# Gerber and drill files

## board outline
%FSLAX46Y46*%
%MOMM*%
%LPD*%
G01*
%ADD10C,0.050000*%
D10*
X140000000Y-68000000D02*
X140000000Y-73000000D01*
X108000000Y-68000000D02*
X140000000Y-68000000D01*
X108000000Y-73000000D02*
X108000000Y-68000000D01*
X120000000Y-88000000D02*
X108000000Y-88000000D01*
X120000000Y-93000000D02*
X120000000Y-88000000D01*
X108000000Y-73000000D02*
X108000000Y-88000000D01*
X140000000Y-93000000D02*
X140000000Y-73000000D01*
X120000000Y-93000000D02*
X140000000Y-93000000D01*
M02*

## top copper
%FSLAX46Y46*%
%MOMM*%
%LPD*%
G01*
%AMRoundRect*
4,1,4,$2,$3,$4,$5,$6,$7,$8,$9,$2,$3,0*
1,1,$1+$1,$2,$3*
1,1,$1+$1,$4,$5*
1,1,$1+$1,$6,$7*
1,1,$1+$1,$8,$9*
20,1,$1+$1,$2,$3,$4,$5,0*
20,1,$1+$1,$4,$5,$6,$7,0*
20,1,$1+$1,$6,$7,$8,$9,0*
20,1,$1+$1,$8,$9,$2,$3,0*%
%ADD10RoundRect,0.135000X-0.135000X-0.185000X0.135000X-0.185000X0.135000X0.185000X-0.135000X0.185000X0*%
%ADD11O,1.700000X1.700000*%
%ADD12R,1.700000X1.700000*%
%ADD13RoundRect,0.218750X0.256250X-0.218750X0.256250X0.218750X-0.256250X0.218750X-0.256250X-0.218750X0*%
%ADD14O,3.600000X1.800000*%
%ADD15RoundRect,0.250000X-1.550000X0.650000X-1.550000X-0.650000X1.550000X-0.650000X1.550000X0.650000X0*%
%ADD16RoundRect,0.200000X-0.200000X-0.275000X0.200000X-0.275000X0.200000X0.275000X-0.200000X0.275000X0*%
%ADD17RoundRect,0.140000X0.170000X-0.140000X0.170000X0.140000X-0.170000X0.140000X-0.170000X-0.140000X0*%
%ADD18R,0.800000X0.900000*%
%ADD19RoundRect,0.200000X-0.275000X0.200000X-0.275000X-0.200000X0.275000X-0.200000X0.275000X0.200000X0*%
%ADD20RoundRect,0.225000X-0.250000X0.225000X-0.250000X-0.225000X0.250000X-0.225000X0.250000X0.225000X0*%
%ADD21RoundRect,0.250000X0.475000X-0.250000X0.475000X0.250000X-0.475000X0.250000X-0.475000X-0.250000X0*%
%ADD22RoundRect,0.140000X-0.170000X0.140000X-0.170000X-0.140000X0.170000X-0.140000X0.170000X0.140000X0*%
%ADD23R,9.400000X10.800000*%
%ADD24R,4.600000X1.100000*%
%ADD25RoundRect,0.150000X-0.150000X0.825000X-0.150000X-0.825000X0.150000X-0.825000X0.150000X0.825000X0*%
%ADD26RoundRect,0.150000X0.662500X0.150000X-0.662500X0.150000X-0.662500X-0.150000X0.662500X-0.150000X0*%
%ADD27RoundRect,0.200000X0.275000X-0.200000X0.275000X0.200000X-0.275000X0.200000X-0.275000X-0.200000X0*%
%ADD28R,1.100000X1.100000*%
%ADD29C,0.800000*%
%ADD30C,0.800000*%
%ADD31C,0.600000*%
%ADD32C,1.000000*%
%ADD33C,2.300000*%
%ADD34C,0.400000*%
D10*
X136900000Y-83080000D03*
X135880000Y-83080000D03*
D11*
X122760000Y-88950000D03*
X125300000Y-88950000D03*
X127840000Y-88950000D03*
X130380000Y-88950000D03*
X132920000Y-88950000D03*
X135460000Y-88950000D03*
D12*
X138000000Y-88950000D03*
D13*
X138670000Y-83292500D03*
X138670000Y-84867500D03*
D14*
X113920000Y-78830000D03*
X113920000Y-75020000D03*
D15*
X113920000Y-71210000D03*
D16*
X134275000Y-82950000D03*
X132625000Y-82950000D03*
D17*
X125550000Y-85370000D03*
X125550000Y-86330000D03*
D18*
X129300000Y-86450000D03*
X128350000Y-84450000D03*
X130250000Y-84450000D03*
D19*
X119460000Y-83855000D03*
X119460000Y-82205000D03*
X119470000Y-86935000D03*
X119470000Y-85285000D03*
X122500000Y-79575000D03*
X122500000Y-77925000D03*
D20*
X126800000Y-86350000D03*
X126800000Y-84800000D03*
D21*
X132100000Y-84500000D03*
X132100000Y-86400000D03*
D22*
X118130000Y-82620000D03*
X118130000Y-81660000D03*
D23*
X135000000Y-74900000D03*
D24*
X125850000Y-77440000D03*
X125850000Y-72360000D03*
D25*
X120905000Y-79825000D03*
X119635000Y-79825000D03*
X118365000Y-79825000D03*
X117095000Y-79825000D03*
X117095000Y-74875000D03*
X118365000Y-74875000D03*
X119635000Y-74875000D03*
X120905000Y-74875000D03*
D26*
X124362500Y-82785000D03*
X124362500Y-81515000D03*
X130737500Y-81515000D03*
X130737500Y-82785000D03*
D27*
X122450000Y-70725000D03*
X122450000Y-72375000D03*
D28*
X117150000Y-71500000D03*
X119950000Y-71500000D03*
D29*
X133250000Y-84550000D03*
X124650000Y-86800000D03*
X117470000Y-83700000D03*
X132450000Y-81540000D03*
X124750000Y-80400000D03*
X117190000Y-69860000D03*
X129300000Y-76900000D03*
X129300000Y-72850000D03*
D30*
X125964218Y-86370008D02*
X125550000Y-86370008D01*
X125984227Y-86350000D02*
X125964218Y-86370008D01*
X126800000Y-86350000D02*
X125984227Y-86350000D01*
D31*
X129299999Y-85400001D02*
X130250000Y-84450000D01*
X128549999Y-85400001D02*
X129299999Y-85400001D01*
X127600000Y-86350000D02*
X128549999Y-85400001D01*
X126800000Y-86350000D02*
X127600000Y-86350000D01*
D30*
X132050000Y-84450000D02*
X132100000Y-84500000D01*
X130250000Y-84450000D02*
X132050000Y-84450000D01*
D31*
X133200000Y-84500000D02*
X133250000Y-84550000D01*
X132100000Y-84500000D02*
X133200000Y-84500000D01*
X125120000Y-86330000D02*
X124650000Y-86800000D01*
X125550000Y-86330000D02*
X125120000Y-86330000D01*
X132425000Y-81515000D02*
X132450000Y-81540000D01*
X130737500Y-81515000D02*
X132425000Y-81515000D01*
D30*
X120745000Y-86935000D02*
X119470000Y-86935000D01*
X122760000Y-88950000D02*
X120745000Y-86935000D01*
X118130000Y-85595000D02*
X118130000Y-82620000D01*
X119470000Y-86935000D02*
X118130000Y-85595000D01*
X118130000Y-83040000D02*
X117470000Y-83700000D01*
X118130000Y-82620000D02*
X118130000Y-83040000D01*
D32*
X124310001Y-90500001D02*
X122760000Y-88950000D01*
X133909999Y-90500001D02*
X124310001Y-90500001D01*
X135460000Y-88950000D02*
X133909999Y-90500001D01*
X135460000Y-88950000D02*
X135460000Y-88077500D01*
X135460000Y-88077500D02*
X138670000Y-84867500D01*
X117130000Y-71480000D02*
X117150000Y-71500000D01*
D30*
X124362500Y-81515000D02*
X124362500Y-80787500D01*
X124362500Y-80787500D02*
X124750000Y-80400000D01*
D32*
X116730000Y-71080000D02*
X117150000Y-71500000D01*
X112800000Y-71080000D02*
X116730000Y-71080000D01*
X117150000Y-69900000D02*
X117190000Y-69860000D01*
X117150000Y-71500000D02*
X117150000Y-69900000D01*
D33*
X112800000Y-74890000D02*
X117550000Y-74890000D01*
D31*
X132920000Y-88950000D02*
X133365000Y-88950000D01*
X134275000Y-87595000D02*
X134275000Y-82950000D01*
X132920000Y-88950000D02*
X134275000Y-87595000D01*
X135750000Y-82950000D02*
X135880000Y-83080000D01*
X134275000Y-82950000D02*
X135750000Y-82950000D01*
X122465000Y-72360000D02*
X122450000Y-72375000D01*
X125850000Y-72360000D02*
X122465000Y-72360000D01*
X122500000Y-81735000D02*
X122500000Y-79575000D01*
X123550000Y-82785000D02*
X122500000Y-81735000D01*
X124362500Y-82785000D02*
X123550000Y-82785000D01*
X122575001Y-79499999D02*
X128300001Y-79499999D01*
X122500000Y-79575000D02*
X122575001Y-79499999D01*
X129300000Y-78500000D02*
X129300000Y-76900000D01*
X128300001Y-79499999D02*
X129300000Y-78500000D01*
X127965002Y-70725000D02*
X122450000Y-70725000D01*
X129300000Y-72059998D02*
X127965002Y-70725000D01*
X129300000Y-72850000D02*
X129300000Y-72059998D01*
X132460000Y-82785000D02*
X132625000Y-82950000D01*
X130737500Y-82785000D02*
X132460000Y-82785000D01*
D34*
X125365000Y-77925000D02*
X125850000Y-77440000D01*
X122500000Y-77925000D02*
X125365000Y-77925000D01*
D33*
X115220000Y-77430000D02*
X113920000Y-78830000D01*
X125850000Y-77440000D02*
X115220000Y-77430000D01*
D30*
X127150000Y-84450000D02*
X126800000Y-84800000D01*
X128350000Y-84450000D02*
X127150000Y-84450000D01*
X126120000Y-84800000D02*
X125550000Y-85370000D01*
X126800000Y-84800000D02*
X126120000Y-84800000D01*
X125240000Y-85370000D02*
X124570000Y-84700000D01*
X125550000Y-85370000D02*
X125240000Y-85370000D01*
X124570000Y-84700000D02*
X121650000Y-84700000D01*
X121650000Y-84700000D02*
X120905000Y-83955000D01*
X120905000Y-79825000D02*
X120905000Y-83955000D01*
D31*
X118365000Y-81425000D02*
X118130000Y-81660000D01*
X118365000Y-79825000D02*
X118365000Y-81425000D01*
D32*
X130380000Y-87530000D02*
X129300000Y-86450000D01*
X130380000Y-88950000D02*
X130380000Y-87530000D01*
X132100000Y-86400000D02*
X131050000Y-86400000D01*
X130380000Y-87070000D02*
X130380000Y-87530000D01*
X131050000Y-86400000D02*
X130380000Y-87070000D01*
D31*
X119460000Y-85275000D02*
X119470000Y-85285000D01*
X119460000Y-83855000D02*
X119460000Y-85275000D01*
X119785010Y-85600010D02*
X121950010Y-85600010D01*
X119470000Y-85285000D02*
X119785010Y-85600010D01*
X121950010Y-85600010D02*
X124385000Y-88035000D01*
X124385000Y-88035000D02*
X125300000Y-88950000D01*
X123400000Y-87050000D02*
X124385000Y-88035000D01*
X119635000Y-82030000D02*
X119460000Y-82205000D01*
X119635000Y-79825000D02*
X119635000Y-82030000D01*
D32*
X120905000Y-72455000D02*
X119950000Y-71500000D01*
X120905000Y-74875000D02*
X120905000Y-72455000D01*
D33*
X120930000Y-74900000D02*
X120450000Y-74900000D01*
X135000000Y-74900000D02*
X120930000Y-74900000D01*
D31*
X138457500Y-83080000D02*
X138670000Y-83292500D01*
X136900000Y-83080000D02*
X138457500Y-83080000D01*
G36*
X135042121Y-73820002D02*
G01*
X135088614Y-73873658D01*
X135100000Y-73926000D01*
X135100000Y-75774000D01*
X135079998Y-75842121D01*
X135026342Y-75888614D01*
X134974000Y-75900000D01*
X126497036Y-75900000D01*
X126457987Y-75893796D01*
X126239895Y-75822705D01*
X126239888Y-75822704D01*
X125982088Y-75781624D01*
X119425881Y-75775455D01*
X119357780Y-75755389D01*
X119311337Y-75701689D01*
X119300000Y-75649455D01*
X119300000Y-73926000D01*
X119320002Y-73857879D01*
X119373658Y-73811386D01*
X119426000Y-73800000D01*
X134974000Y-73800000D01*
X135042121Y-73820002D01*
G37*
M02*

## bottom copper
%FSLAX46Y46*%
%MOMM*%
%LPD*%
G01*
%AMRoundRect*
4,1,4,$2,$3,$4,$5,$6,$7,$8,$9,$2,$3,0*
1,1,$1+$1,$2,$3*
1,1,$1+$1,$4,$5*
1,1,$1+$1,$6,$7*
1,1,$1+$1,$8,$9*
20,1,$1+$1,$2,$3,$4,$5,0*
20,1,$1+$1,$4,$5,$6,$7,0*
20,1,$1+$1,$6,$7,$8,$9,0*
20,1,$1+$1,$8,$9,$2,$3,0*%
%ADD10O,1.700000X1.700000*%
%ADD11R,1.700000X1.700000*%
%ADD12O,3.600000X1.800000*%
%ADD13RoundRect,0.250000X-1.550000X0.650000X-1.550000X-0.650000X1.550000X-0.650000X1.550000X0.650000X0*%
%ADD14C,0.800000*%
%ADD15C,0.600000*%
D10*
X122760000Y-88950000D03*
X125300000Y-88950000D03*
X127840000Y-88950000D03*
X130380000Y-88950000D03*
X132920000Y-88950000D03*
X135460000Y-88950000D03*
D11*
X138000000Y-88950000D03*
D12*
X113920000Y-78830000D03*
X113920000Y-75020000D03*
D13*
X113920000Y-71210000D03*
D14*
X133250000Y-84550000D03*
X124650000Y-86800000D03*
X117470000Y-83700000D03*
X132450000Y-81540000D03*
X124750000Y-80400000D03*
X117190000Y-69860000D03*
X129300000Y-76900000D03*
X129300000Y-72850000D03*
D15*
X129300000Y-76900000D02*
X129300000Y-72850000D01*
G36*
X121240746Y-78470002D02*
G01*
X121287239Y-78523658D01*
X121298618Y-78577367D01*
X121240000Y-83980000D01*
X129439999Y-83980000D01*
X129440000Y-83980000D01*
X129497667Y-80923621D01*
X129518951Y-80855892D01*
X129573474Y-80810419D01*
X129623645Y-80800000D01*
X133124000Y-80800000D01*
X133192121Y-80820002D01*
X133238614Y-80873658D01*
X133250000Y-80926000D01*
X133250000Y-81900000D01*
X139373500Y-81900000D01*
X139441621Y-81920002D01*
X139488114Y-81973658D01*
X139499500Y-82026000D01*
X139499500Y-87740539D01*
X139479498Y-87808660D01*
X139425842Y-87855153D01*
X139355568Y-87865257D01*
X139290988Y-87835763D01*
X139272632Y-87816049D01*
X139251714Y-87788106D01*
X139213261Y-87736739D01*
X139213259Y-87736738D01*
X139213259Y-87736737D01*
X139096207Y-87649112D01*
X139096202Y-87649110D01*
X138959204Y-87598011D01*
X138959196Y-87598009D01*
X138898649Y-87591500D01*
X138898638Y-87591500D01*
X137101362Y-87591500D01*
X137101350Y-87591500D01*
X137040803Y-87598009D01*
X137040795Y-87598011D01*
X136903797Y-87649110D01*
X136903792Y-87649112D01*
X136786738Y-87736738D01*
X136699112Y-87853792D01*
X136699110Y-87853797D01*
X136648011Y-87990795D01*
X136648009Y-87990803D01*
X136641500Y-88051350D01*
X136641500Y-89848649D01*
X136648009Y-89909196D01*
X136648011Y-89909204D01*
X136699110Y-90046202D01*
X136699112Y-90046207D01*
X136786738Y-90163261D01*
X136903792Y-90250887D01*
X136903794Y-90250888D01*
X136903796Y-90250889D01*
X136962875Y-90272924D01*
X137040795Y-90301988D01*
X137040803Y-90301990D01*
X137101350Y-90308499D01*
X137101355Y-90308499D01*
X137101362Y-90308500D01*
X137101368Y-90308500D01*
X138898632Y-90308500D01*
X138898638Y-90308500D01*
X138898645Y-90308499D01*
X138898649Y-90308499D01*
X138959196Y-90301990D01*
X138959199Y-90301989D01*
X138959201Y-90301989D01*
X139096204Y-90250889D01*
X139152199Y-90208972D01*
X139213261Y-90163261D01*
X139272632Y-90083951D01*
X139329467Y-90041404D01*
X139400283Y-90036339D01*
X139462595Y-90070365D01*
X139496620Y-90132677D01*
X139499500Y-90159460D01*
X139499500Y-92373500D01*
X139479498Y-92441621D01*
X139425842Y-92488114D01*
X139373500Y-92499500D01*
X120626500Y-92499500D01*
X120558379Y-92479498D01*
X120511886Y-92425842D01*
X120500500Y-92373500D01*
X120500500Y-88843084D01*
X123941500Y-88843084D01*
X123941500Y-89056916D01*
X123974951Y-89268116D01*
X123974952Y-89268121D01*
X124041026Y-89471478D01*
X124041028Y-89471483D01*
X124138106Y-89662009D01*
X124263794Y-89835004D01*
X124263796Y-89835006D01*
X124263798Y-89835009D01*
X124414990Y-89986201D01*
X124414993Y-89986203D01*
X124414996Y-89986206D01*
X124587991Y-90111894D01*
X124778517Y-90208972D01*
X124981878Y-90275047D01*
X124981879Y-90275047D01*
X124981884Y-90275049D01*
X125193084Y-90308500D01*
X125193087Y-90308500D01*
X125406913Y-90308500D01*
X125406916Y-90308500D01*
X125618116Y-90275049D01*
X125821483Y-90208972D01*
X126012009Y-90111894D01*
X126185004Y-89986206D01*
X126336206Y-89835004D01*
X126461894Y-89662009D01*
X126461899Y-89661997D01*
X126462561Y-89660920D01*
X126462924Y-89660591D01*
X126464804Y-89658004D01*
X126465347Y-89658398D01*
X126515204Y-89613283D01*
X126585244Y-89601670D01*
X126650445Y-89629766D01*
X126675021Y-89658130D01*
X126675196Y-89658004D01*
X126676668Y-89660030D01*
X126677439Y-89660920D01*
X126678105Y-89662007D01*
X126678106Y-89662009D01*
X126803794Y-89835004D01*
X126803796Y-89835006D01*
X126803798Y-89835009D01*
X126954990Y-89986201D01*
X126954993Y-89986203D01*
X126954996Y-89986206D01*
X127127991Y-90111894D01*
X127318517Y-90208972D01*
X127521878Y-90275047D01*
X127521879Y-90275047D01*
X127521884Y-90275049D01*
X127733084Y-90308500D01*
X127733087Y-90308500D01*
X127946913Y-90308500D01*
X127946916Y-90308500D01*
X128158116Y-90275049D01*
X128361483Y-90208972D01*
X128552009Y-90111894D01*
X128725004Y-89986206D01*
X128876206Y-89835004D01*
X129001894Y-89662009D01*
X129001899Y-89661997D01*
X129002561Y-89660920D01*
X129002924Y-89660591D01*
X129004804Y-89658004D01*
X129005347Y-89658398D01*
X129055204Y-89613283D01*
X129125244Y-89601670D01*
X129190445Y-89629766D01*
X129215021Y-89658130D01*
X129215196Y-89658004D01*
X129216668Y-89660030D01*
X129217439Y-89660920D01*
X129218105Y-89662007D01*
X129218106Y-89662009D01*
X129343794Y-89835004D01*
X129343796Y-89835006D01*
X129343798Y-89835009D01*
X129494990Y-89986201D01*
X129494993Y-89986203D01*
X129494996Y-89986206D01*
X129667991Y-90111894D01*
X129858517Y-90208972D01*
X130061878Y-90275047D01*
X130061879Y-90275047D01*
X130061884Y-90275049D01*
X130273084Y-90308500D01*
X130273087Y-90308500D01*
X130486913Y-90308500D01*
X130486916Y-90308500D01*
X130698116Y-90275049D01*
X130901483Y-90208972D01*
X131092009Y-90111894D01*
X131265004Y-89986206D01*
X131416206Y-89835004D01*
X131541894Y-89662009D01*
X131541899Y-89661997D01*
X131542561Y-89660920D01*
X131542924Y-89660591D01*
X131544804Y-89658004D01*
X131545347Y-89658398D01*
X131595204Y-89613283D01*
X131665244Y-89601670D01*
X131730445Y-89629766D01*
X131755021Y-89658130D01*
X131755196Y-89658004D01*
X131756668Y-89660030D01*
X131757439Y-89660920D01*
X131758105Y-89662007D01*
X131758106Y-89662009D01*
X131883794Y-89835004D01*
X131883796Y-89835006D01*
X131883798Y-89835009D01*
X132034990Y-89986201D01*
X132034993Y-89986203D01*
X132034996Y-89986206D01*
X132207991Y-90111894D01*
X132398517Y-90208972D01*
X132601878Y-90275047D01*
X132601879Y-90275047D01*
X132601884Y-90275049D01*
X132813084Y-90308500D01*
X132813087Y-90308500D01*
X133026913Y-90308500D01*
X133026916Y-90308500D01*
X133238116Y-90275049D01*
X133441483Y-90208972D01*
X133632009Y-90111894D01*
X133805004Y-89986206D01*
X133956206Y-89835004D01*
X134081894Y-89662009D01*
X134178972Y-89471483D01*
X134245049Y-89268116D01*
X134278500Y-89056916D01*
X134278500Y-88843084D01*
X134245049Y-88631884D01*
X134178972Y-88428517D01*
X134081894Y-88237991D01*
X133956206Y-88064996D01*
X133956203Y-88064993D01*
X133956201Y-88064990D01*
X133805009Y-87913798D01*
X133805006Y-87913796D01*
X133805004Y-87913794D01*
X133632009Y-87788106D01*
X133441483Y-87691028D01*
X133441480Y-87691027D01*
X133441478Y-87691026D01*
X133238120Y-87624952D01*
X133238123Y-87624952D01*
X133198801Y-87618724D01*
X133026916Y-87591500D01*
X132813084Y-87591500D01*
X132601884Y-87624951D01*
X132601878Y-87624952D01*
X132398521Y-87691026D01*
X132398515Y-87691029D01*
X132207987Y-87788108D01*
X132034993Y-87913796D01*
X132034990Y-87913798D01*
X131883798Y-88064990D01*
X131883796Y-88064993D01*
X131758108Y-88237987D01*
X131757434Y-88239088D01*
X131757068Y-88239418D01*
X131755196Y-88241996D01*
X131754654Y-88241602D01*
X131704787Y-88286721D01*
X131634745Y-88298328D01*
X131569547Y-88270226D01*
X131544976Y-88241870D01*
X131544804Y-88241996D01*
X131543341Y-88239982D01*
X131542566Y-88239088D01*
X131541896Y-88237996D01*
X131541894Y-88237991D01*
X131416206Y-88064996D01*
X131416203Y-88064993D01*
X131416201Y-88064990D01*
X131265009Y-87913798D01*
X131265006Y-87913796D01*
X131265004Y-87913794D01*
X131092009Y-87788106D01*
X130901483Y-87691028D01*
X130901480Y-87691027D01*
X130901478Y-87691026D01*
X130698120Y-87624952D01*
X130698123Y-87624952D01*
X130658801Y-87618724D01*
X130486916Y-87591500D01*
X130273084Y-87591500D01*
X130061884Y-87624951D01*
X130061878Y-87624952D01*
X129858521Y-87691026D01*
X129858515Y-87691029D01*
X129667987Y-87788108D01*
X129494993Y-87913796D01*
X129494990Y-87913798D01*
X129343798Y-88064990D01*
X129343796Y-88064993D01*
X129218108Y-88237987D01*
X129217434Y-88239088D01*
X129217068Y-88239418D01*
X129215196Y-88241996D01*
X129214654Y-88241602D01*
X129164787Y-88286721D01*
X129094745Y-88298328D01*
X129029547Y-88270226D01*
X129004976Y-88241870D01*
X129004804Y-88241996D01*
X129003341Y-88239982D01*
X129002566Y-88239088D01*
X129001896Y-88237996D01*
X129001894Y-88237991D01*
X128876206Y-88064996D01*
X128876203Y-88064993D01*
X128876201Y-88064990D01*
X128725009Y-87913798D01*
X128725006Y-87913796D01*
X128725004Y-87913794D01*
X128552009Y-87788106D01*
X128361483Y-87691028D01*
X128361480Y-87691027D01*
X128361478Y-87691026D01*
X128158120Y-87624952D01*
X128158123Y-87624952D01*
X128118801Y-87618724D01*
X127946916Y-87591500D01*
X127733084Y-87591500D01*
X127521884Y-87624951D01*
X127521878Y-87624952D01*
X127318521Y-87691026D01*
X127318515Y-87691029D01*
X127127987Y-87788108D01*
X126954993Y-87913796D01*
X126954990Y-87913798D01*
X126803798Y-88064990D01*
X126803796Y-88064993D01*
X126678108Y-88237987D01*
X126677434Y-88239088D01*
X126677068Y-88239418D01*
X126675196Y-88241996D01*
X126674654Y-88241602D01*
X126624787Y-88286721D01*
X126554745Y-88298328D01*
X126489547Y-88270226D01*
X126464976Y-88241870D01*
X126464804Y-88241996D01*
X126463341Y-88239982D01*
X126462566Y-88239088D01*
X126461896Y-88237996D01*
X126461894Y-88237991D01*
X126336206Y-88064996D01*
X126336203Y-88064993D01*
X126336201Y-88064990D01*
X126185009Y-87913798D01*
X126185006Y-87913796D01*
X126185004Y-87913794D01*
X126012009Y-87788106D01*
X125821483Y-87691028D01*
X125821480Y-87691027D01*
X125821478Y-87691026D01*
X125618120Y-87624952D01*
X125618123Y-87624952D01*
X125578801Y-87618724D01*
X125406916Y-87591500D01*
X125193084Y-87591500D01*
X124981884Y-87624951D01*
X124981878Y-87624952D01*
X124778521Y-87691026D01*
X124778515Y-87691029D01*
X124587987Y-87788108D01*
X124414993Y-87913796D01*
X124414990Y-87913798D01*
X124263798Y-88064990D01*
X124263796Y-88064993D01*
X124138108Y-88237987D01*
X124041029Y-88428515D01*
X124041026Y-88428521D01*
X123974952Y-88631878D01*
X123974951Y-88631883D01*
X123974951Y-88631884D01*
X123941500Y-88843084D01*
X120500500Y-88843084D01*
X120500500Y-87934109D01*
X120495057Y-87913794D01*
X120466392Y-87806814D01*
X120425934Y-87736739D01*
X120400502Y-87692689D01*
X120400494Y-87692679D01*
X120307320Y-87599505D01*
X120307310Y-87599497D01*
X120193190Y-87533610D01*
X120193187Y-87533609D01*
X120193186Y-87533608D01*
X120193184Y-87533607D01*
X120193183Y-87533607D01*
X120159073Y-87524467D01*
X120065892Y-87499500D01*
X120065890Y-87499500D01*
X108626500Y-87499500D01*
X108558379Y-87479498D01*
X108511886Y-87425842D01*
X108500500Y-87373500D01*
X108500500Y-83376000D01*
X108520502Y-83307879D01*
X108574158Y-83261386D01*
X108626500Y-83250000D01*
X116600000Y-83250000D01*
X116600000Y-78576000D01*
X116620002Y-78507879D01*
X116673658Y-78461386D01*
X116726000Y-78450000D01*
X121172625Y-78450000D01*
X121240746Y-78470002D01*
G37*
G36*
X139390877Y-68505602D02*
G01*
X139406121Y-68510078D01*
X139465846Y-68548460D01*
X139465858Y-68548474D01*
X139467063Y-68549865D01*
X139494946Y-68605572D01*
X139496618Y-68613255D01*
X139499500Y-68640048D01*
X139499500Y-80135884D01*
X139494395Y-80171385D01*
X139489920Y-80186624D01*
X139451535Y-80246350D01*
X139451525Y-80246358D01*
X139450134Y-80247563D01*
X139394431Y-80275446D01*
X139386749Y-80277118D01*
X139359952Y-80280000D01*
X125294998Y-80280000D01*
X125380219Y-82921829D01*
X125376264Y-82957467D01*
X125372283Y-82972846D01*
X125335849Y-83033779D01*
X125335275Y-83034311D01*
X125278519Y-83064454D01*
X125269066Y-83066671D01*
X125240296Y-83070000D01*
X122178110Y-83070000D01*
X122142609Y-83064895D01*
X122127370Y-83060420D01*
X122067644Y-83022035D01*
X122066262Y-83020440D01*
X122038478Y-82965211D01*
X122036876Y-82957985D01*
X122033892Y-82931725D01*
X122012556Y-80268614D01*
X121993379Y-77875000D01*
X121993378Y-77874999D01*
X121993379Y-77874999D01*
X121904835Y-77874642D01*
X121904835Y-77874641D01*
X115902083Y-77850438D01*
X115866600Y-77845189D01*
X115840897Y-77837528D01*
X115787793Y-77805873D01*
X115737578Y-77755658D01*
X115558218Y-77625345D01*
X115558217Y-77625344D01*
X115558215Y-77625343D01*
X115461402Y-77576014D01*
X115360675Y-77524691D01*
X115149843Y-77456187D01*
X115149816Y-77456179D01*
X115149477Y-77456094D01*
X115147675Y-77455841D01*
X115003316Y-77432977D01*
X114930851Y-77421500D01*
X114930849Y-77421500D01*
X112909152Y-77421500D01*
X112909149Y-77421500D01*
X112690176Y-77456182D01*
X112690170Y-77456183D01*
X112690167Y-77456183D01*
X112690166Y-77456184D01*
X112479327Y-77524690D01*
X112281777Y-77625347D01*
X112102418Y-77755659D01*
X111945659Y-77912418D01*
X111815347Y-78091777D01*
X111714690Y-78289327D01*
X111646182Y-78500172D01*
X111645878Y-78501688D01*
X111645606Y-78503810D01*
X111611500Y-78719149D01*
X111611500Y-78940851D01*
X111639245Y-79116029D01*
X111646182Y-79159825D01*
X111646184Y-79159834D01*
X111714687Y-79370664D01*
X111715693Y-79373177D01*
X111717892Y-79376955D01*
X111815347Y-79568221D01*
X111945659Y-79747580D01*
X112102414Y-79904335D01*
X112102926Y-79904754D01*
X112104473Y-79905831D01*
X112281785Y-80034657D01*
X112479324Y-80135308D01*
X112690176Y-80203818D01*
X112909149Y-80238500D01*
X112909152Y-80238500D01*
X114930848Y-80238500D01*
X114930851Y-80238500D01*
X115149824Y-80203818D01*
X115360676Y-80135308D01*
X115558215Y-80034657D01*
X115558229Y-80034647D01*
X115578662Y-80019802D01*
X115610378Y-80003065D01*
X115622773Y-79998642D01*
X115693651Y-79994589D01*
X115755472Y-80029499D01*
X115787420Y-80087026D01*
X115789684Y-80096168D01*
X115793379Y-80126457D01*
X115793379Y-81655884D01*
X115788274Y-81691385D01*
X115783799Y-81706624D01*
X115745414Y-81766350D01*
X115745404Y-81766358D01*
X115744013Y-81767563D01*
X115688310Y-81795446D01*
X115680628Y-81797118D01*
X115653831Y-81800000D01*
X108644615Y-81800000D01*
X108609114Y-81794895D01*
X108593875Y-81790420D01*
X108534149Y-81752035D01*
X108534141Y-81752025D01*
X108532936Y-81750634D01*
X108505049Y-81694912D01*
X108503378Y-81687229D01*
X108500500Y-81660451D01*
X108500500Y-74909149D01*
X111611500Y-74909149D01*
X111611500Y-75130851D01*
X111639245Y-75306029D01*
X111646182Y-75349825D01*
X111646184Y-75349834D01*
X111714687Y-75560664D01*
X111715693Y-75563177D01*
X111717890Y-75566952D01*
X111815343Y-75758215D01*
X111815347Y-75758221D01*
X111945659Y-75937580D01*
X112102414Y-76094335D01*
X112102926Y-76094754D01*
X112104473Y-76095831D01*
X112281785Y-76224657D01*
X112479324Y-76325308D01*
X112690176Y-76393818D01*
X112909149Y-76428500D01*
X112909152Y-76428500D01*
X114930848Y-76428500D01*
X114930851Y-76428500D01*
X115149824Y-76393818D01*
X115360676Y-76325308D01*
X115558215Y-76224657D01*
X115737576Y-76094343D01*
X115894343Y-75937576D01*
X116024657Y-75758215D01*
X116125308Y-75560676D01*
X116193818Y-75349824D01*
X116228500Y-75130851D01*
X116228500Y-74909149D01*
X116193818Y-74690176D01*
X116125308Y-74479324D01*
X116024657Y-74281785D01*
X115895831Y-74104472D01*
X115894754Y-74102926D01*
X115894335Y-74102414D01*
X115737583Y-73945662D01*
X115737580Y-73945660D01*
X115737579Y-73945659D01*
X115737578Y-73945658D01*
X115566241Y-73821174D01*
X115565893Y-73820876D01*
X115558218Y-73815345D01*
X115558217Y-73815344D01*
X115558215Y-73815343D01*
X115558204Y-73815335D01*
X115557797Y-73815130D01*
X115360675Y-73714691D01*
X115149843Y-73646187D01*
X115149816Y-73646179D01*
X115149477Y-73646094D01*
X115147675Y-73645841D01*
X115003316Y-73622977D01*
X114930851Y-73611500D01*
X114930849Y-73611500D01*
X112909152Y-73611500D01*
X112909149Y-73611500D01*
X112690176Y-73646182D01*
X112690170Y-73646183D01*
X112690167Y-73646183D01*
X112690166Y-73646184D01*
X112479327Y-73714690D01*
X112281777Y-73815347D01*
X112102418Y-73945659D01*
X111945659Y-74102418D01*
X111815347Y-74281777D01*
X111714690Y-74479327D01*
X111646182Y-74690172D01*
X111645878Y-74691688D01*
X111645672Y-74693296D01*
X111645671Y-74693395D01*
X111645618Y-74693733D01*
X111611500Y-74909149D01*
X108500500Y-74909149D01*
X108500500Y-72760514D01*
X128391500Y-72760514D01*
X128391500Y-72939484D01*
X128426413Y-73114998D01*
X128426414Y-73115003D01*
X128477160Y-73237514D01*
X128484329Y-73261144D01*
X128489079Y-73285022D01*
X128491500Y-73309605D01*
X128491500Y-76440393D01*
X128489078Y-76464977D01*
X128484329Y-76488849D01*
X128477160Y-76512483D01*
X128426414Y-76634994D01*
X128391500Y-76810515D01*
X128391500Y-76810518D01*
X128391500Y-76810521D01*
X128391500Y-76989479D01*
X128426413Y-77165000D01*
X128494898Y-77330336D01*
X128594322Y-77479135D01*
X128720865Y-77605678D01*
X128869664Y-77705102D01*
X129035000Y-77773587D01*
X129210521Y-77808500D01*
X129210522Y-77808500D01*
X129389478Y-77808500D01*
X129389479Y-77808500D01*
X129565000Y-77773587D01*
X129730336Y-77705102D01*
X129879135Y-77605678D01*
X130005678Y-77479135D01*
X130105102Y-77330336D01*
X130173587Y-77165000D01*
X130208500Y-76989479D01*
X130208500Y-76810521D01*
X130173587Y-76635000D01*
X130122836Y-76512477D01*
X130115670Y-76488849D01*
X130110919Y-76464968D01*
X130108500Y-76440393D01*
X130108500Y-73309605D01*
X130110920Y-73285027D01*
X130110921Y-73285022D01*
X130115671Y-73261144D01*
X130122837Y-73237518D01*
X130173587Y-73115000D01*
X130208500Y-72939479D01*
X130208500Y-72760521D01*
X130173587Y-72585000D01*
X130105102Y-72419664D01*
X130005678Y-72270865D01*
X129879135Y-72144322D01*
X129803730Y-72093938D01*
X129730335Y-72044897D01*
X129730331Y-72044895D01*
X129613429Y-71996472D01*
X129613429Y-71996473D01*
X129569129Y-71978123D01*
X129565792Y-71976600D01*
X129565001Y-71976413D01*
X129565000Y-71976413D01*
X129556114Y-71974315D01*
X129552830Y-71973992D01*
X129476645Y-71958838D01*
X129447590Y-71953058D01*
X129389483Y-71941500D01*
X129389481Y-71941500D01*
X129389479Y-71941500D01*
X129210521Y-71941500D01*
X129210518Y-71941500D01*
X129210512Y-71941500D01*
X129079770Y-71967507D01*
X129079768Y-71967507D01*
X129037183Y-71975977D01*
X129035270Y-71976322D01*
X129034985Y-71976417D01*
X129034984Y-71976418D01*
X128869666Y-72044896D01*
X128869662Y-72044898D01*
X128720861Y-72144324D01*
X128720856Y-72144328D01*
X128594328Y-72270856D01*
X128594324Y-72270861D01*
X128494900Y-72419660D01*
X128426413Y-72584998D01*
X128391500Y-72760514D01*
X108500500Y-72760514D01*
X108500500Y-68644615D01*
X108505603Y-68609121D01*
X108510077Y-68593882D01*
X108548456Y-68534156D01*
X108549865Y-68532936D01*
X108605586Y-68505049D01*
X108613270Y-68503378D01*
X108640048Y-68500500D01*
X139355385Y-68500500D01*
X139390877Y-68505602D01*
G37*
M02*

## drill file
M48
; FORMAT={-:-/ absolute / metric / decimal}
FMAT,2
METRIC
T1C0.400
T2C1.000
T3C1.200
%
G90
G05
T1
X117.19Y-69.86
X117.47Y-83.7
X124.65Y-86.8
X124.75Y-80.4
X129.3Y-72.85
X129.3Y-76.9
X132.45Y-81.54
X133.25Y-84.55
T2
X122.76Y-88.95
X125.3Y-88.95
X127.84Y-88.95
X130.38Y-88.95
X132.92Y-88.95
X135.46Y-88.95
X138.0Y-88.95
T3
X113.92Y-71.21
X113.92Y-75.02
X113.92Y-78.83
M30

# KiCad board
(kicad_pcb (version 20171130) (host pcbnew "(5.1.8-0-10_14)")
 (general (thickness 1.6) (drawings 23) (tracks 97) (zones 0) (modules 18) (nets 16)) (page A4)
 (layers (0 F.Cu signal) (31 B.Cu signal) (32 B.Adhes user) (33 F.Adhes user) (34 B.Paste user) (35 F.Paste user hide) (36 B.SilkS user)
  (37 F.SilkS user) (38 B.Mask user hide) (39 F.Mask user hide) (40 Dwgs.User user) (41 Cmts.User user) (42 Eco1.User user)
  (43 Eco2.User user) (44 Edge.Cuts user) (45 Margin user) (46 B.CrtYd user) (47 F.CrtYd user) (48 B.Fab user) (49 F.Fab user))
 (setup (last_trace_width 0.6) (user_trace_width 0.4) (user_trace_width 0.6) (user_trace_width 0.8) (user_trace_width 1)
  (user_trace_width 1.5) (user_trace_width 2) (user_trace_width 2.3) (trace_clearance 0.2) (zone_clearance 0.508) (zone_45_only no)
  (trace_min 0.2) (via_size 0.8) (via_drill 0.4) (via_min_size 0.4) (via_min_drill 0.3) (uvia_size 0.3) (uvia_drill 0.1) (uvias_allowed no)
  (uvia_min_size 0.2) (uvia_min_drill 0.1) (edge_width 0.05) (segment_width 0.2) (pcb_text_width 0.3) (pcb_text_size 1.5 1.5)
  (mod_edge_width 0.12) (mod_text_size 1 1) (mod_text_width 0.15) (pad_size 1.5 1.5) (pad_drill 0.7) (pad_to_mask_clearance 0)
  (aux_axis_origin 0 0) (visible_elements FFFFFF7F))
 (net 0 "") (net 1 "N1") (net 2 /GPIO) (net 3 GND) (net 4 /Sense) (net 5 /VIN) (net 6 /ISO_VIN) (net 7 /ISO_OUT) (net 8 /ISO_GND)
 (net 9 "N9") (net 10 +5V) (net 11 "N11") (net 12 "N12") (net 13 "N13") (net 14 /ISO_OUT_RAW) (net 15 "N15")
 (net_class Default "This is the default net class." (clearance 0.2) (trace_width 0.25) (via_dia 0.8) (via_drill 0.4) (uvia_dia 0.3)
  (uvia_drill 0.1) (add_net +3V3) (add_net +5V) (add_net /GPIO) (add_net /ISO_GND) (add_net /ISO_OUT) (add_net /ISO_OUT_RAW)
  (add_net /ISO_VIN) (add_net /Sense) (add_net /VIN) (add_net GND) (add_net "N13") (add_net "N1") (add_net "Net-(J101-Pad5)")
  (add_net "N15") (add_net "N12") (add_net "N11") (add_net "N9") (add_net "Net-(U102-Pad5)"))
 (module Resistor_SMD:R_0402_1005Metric (layer F.Cu) (at 136.39 83.08)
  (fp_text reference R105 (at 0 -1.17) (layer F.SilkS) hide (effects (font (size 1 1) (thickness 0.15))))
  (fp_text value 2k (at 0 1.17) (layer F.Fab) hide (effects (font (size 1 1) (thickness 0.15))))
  (pad 2 smd roundrect (at 0.51 0) (size 0.54 0.64) (layers F.Cu F.Paste F.Mask) (roundrect_rratio 0.25) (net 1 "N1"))
  (pad 1 smd roundrect (at -0.51 0) (size 0.54 0.64) (layers F.Cu F.Paste F.Mask) (roundrect_rratio 0.25) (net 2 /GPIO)))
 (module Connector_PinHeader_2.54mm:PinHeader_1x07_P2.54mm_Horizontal (layer F.Cu) (at 138 88.95 270)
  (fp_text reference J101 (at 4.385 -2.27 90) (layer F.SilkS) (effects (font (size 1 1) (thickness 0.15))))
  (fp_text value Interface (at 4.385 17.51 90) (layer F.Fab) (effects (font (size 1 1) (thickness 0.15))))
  (pad 7 thru_hole oval (at 0 15.24 270) (size 1.7 1.7) (drill 1) (layers *.Cu *.Mask) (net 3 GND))
  (pad 6 thru_hole oval (at 0 12.7 270) (size 1.7 1.7) (drill 1) (layers *.Cu *.Mask) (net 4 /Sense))
  (pad 5 thru_hole oval (at 0 10.16 270) (size 1.7 1.7) (drill 1) (layers *.Cu *.Mask))
  (pad 4 thru_hole oval (at 0 7.62 270) (size 1.7 1.7) (drill 1) (layers *.Cu *.Mask) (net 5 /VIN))
  (pad 3 thru_hole oval (at 0 5.08 270) (size 1.7 1.7) (drill 1) (layers *.Cu *.Mask) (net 2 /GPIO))
  (pad 2 thru_hole oval (at 0 2.54 270) (size 1.7 1.7) (drill 1) (layers *.Cu *.Mask) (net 3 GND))
  (pad 1 thru_hole rect (at 0 0 270) (size 1.7 1.7) (drill 1) (layers *.Cu *.Mask)))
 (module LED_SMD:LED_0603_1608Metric (layer F.Cu) (at 138.67 84.08 90)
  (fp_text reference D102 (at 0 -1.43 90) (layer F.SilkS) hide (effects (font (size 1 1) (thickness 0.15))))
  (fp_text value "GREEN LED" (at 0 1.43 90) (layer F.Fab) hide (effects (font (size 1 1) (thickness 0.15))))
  (pad 2 smd roundrect (at 0.7875 0 90) (size 0.875 0.95) (layers F.Cu F.Paste F.Mask) (roundrect_rratio 0.25) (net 1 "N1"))
  (pad 1 smd roundrect (at -0.7875 0 90) (size 0.875 0.95) (layers F.Cu F.Paste F.Mask) (roundrect_rratio 0.25) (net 3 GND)))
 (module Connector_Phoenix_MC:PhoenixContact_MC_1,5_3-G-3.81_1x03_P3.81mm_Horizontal (layer F.Cu) (at 113.92 71.21 270)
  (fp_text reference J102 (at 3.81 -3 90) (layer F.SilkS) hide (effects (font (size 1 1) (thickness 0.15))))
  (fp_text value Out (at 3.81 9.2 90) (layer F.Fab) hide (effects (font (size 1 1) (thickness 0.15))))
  (pad 3 thru_hole oval (at 7.62 0 270) (size 1.8 3.6) (drill 1.2) (layers *.Cu *.Mask) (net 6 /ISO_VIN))
  (pad 2 thru_hole oval (at 3.81 0 270) (size 1.8 3.6) (drill 1.2) (layers *.Cu *.Mask) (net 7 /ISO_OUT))
  (pad 1 thru_hole roundrect (at 0 0 270) (size 1.8 3.6) (drill 1.2) (layers *.Cu *.Mask) (roundrect_rratio 0.1388888888888889)
   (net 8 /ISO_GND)))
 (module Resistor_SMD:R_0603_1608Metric (layer F.Cu) (at 133.45 82.95)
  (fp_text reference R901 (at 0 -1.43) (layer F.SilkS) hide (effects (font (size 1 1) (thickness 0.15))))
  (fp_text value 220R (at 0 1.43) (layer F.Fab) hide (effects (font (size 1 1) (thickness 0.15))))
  (pad 2 smd roundrect (at 0.825 0) (size 0.8 0.95) (layers F.Cu F.Paste F.Mask) (roundrect_rratio 0.25) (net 2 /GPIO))
  (pad 1 smd roundrect (at -0.825 0) (size 0.8 0.95) (layers F.Cu F.Paste F.Mask) (roundrect_rratio 0.25) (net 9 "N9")))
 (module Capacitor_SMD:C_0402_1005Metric (layer F.Cu) (at 125.55 85.85 90)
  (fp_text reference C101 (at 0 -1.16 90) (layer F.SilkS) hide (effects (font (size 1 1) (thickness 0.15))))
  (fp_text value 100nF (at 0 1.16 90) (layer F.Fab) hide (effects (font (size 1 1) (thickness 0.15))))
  (pad 2 smd roundrect (at 0.48 0 90) (size 0.56 0.62) (layers F.Cu F.Paste F.Mask) (roundrect_rratio 0.25) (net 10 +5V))
  (pad 1 smd roundrect (at -0.48 0 90) (size 0.56 0.62) (layers F.Cu F.Paste F.Mask) (roundrect_rratio 0.25) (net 3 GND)))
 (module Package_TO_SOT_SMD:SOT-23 (layer F.Cu) (at 129.3 85.45 270)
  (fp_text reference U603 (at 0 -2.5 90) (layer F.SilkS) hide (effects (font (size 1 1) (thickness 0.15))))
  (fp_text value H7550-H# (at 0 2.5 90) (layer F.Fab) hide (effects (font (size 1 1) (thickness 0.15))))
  (pad 3 smd rect (at 1 0 270) (size 0.9 0.8) (layers F.Cu F.Paste F.Mask) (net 5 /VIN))
  (pad 2 smd rect (at -1 0.95 270) (size 0.9 0.8) (layers F.Cu F.Paste F.Mask) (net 10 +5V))
  (pad 1 smd rect (at -1 -0.95 270) (size 0.9 0.8) (layers F.Cu F.Paste F.Mask) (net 3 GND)))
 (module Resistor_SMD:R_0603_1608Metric (layer F.Cu) (at 119.46 83.03 270)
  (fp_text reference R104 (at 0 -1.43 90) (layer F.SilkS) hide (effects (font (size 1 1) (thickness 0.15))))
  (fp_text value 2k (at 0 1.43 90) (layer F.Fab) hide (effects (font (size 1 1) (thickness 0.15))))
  (pad 2 smd roundrect (at 0.825 0 270) (size 0.8 0.95) (layers F.Cu F.Paste F.Mask) (roundrect_rratio 0.25) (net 4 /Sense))
  (pad 1 smd roundrect (at -0.825 0 270) (size 0.8 0.95) (layers F.Cu F.Paste F.Mask) (roundrect_rratio 0.25) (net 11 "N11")))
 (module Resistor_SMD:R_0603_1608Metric (layer F.Cu) (at 119.47 86.11 270)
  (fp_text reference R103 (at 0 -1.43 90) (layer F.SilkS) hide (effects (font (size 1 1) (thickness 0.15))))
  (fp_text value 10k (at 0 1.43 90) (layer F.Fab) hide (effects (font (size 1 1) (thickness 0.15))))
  (pad 2 smd roundrect (at 0.825 0 270) (size 0.8 0.95) (layers F.Cu F.Paste F.Mask) (roundrect_rratio 0.25) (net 3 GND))
  (pad 1 smd roundrect (at -0.825 0 270) (size 0.8 0.95) (layers F.Cu F.Paste F.Mask) (roundrect_rratio 0.25) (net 4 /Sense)))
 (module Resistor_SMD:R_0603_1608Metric (layer F.Cu) (at 122.5 78.75 270)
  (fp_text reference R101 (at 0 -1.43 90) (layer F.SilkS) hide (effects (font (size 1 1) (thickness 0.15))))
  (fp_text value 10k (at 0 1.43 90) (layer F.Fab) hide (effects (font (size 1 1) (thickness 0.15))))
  (pad 2 smd roundrect (at 0.825 0 270) (size 0.8 0.95) (layers F.Cu F.Paste F.Mask) (roundrect_rratio 0.25) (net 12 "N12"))
  (pad 1 smd roundrect (at -0.825 0 270) (size 0.8 0.95) (layers F.Cu F.Paste F.Mask) (roundrect_rratio 0.25) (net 6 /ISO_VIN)))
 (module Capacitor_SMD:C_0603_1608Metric (layer F.Cu) (at 126.8 85.575 270)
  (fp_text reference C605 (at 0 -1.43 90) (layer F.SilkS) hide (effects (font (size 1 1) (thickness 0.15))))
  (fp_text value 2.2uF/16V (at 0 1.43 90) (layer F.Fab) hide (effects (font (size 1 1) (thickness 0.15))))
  (pad 2 smd roundrect (at 0.775 0 270) (size 0.9 0.95) (layers F.Cu F.Paste F.Mask) (roundrect_rratio 0.25) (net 3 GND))
  (pad 1 smd roundrect (at -0.775 0 270) (size 0.9 0.95) (layers F.Cu F.Paste F.Mask) (roundrect_rratio 0.25) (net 10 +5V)))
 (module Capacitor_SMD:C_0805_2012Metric (layer F.Cu) (at 132.1 85.45 90)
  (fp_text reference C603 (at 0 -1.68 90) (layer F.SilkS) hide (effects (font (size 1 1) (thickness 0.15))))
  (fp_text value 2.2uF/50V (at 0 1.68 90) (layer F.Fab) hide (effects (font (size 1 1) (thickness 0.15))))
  (pad 2 smd roundrect (at 0.95 0 90) (size 1 1.45) (layers F.Cu F.Paste F.Mask) (roundrect_rratio 0.25) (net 3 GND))
  (pad 1 smd roundrect (at -0.95 0 90) (size 1 1.45) (layers F.Cu F.Paste F.Mask) (roundrect_rratio 0.25) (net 5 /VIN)))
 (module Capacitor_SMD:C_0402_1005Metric (layer F.Cu) (at 118.13 82.14 270)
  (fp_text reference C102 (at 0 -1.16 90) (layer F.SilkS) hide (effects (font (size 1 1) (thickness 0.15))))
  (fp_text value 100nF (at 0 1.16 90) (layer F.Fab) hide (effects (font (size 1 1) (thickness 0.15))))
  (pad 2 smd roundrect (at 0.48 0 270) (size 0.56 0.62) (layers F.Cu F.Paste F.Mask) (roundrect_rratio 0.25) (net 3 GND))
  (pad 1 smd roundrect (at -0.48 0 270) (size 0.56 0.62) (layers F.Cu F.Paste F.Mask) (roundrect_rratio 0.25) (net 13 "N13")))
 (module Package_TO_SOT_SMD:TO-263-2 (layer F.Cu) (at 131.625 74.9)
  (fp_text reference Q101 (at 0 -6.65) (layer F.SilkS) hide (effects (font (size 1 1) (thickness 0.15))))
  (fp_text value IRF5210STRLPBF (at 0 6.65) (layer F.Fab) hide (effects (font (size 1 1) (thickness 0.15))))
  (pad "" smd rect (at 0.95 2.775) (size 4.55 5.25) (layers F.Paste))
  (pad "" smd rect (at 5.8 -2.775) (size 4.55 5.25) (layers F.Paste))
  (pad "" smd rect (at 0.95 -2.775) (size 4.55 5.25) (layers F.Paste))
  (pad "" smd rect (at 5.8 2.775) (size 4.55 5.25) (layers F.Paste))
  (pad 2 smd rect (at 3.375 0) (size 9.4 10.8) (layers F.Cu F.Mask) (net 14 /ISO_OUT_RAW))
  (pad 3 smd rect (at -5.775 2.54) (size 4.6 1.1) (layers F.Cu F.Paste F.Mask) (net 6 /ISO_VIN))
  (pad 1 smd rect (at -5.775 -2.54) (size 4.6 1.1) (layers F.Cu F.Paste F.Mask) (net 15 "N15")))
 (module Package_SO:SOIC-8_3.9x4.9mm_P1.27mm (layer F.Cu) (at 119 77.35 270)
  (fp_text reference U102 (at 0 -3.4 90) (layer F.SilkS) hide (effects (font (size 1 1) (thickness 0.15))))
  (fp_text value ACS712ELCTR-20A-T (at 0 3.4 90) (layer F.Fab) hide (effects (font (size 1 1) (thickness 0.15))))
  (pad 8 smd roundrect (at 2.475 -1.905 270) (size 1.95 0.6) (layers F.Cu F.Paste F.Mask) (roundrect_rratio 0.25) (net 10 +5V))
  (pad 7 smd roundrect (at 2.475 -0.635 270) (size 1.95 0.6) (layers F.Cu F.Paste F.Mask) (roundrect_rratio 0.25) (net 11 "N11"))
  (pad 6 smd roundrect (at 2.475 0.635 270) (size 1.95 0.6) (layers F.Cu F.Paste F.Mask) (roundrect_rratio 0.25) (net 13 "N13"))
  (pad 5 smd roundrect (at 2.475 1.905 270) (size 1.95 0.6) (layers F.Cu F.Paste F.Mask) (roundrect_rratio 0.25))
  (pad 4 smd roundrect (at -2.475 1.905 270) (size 1.95 0.6) (layers F.Cu F.Paste F.Mask) (roundrect_rratio 0.25) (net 7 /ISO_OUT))
  (pad 3 smd roundrect (at -2.475 0.635 270) (size 1.95 0.6) (layers F.Cu F.Paste F.Mask) (roundrect_rratio 0.25) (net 7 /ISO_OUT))
  (pad 2 smd roundrect (at -2.475 -0.635 270) (size 1.95 0.6) (layers F.Cu F.Paste F.Mask) (roundrect_rratio 0.25) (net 14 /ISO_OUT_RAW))
  (pad 1 smd roundrect (at -2.475 -1.905 270) (size 1.95 0.6) (layers F.Cu F.Paste F.Mask) (roundrect_rratio 0.25) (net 14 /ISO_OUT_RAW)))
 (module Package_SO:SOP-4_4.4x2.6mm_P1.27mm (layer F.Cu) (at 127.55 82.15 180)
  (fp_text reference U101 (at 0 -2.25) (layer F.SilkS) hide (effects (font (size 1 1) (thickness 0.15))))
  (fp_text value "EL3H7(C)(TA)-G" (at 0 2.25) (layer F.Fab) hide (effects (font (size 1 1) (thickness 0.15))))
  (pad 4 smd roundrect (at 3.1875 -0.635 180) (size 1.625 0.6) (layers F.Cu F.Paste F.Mask) (roundrect_rratio 0.25) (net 12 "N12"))
  (pad 3 smd roundrect (at 3.1875 0.635 180) (size 1.625 0.6) (layers F.Cu F.Paste F.Mask) (roundrect_rratio 0.25) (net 8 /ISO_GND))
  (pad 2 smd roundrect (at -3.1875 0.635 180) (size 1.625 0.6) (layers F.Cu F.Paste F.Mask) (roundrect_rratio 0.25) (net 3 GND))
  (pad 1 smd roundrect (at -3.1875 -0.635 180) (size 1.625 0.6) (layers F.Cu F.Paste F.Mask) (roundrect_rratio 0.25) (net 9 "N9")))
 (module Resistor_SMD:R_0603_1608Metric (layer F.Cu) (at 122.45 71.55 90)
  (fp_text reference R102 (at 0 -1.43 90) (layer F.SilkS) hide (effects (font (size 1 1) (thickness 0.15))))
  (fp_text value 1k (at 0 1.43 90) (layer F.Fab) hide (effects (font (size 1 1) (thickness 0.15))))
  (pad 2 smd roundrect (at 0.825 0 90) (size 0.8 0.95) (layers F.Cu F.Paste F.Mask) (roundrect_rratio 0.25) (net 12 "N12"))
  (pad 1 smd roundrect (at -0.825 0 90) (size 0.8 0.95) (layers F.Cu F.Paste F.Mask) (roundrect_rratio 0.25) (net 15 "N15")))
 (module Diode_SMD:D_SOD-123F (layer F.Cu) (at 118.55 71.5 180)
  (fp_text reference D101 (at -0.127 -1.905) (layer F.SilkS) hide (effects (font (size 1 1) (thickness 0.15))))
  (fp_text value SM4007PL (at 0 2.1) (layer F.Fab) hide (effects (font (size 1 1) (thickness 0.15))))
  (pad 2 smd rect (at 1.4 0 180) (size 1.1 1.1) (layers F.Cu F.Paste F.Mask) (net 8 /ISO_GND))
  (pad 1 smd rect (at -1.4 0 180) (size 1.1 1.1) (layers F.Cu F.Paste F.Mask) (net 14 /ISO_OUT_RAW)))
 (gr_line (start 140 68) (end 140 73) (layer Edge.Cuts) (width 0.05))
 (gr_line (start 108 68) (end 140 68) (layer Edge.Cuts) (width 0.05))
 (gr_line (start 108 73) (end 108 68) (layer Edge.Cuts) (width 0.05))
 (gr_line (start 120 88) (end 108 88) (layer Edge.Cuts) (width 0.05))
 (gr_line (start 120 93) (end 120 88) (layer Edge.Cuts) (width 0.05))
 (gr_line (start 108 73) (end 108 88) (layer Edge.Cuts) (width 0.05))
 (gr_line (start 140 93) (end 140 73) (layer Edge.Cuts) (width 0.05))
 (gr_line (start 120 93) (end 140 93) (layer Edge.Cuts) (width 0.05))
 (segment (start 125.964218 86.370008) (end 125.55 86.370008) (width 0.8) (layer F.Cu) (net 3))
 (segment (start 125.984227 86.35) (end 125.964218 86.370008) (width 0.8) (layer F.Cu) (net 3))
 (segment (start 126.8 86.35) (end 125.984227 86.35) (width 0.8) (layer F.Cu) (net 3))
 (segment (start 129.299999 85.400001) (end 130.25 84.45) (width 0.6) (layer F.Cu) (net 3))
 (segment (start 128.549999 85.400001) (end 129.299999 85.400001) (width 0.6) (layer F.Cu) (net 3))
 (segment (start 127.6 86.35) (end 128.549999 85.400001) (width 0.6) (layer F.Cu) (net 3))
 (segment (start 126.8 86.35) (end 127.6 86.35) (width 0.6) (layer F.Cu) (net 3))
 (segment (start 132.05 84.45) (end 132.1 84.5) (width 0.8) (layer F.Cu) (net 3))
 (segment (start 130.25 84.45) (end 132.05 84.45) (width 0.8) (layer F.Cu) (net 3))
 (via (at 133.25 84.55) (size 0.8) (drill 0.4) (layers F.Cu B.Cu) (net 3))
 (segment (start 133.2 84.5) (end 133.25 84.55) (width 0.6) (layer F.Cu) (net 3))
 (segment (start 132.1 84.5) (end 133.2 84.5) (width 0.6) (layer F.Cu) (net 3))
 (segment (start 125.12 86.33) (end 124.65 86.8) (width 0.6) (layer F.Cu) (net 3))
 (via (at 124.65 86.8) (size 0.8) (drill 0.4) (layers F.Cu B.Cu) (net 3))
 (segment (start 125.55 86.33) (end 125.12 86.33) (width 0.6) (layer F.Cu) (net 3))
 (via (at 117.47 83.7) (size 0.8) (drill 0.4) (layers F.Cu B.Cu) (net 3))
 (via (at 132.45 81.54) (size 0.8) (drill 0.4) (layers F.Cu B.Cu) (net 3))
 (segment (start 132.425 81.515) (end 132.45 81.54) (width 0.6) (layer F.Cu) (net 3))
 (segment (start 130.7375 81.515) (end 132.425 81.515) (width 0.6) (layer F.Cu) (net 3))
 (segment (start 120.745 86.935) (end 119.47 86.935) (width 0.8) (layer F.Cu) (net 3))
 (segment (start 122.76 88.95) (end 120.745 86.935) (width 0.8) (layer F.Cu) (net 3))
 (segment (start 118.13 85.595) (end 118.13 82.62) (width 0.8) (layer F.Cu) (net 3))
 (segment (start 119.47 86.935) (end 118.13 85.595) (width 0.8) (layer F.Cu) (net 3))
 (segment (start 118.13 83.04) (end 117.47 83.7) (width 0.8) (layer F.Cu) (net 3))
 (segment (start 118.13 82.62) (end 118.13 83.04) (width 0.8) (layer F.Cu) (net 3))
 (segment (start 124.310001 90.500001) (end 122.76 88.95) (width 1) (layer F.Cu) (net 3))
 (segment (start 133.909999 90.500001) (end 124.310001 90.500001) (width 1) (layer F.Cu) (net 3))
 (segment (start 135.46 88.95) (end 133.909999 90.500001) (width 1) (layer F.Cu) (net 3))
 (segment (start 135.46 88.95) (end 135.46 88.0775) (width 1) (layer F.Cu) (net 3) (status 1000000))
 (segment (start 135.46 88.0775) (end 138.67 84.8675) (width 1) (layer F.Cu) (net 3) (status 1000000))
 (via (at 124.75 80.4) (size 0.8) (drill 0.4) (layers F.Cu B.Cu) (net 8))
 (via (at 117.19 69.86) (size 0.8) (drill 0.4) (layers F.Cu B.Cu) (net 8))
 (segment (start 117.13 71.48) (end 117.15 71.5) (width 1) (layer F.Cu) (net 8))
 (segment (start 124.3625 81.515) (end 124.3625 80.7875) (width 0.8) (layer F.Cu) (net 8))
 (segment (start 124.3625 80.7875) (end 124.75 80.4) (width 0.8) (layer F.Cu) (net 8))
 (segment (start 116.73 71.08) (end 117.15 71.5) (width 1) (layer F.Cu) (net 8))
 (segment (start 112.8 71.08) (end 116.73 71.08) (width 1) (layer F.Cu) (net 8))
 (segment (start 117.15 69.9) (end 117.19 69.86) (width 1) (layer F.Cu) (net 8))
 (segment (start 117.15 71.5) (end 117.15 69.9) (width 1) (layer F.Cu) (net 8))
 (segment (start 112.8 74.89) (end 117.55 74.89) (width 2.3) (layer F.Cu) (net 7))
 (segment (start 132.92 88.95) (end 133.365 88.95) (width 0.6) (layer F.Cu) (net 2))
 (segment (start 134.275 87.595) (end 134.275 82.95) (width 0.6) (layer F.Cu) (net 2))
 (segment (start 132.92 88.95) (end 134.275 87.595) (width 0.6) (layer F.Cu) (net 2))
 (segment (start 135.75 82.95) (end 135.88 83.08) (width 0.6) (layer F.Cu) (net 2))
 (segment (start 134.275 82.95) (end 135.75 82.95) (width 0.6) (layer F.Cu) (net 2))
 (segment (start 122.465 72.36) (end 122.45 72.375) (width 0.6) (layer F.Cu) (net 15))
 (segment (start 125.85 72.36) (end 122.465 72.36) (width 0.6) (layer F.Cu) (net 15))
 (segment (start 122.5 81.735) (end 122.5 79.575) (width 0.6) (layer F.Cu) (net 12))
 (segment (start 123.55 82.785) (end 122.5 81.735) (width 0.6) (layer F.Cu) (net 12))
 (segment (start 124.3625 82.785) (end 123.55 82.785) (width 0.6) (layer F.Cu) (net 12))
 (segment (start 122.575001 79.499999) (end 128.300001 79.499999) (width 0.6) (layer F.Cu) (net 12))
 (segment (start 122.5 79.575) (end 122.575001 79.499999) (width 0.6) (layer F.Cu) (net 12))
 (via (at 129.3 76.9) (size 0.8) (drill 0.4) (layers F.Cu B.Cu) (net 12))
 (segment (start 129.3 78.5) (end 129.3 76.9) (width 0.6) (layer F.Cu) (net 12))
 (segment (start 128.300001 79.499999) (end 129.3 78.5) (width 0.6) (layer F.Cu) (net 12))
 (via (at 129.3 72.85) (size 0.8) (drill 0.4) (layers F.Cu B.Cu) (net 12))
 (segment (start 129.3 76.9) (end 129.3 72.85) (width 0.6) (layer B.Cu) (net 12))
 (segment (start 127.965002 70.725) (end 122.45 70.725) (width 0.6) (layer F.Cu) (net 12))
 (segment (start 129.3 72.059998) (end 127.965002 70.725) (width 0.6) (layer F.Cu) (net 12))
 (segment (start 129.3 72.85) (end 129.3 72.059998) (width 0.6) (layer F.Cu) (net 12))
 (segment (start 132.46 82.785) (end 132.625 82.95) (width 0.6) (layer F.Cu) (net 9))
 (segment (start 130.7375 82.785) (end 132.46 82.785) (width 0.6) (layer F.Cu) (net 9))
 (segment (start 125.365 77.925) (end 125.85 77.44) (width 0.4) (layer F.Cu) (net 6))
 (segment (start 122.5 77.925) (end 125.365 77.925) (width 0.4) (layer F.Cu) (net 6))
 (segment (start 115.22 77.43) (end 113.92 78.83) (width 2.3) (layer F.Cu) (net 6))
 (segment (start 125.85 77.44) (end 115.22 77.43) (width 2.3) (layer F.Cu) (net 6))
 (segment (start 127.15 84.45) (end 126.8 84.8) (width 0.8) (layer F.Cu) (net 10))
 (segment (start 128.35 84.45) (end 127.15 84.45) (width 0.8) (layer F.Cu) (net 10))
 (segment (start 126.12 84.8) (end 125.55 85.37) (width 0.8) (layer F.Cu) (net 10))
 (segment (start 126.8 84.8) (end 126.12 84.8) (width 0.8) (layer F.Cu) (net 10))
 (segment (start 125.24 85.37) (end 124.57 84.7) (width 0.8) (layer F.Cu) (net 10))
 (segment (start 125.55 85.37) (end 125.24 85.37) (width 0.8) (layer F.Cu) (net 10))
 (segment (start 124.57 84.7) (end 121.65 84.7) (width 0.8) (layer F.Cu) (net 10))
 (segment (start 121.65 84.7) (end 120.905 83.955) (width 0.8) (layer F.Cu) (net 10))
 (segment (start 120.905 79.825) (end 120.905 83.955) (width 0.8) (layer F.Cu) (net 10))
 (segment (start 118.365 81.425) (end 118.13 81.66) (width 0.6) (layer F.Cu) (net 13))
 (segment (start 118.365 79.825) (end 118.365 81.425) (width 0.6) (layer F.Cu) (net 13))
 (segment (start 130.38 87.53) (end 129.3 86.45) (width 1) (layer F.Cu) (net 5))
 (segment (start 130.38 88.95) (end 130.38 87.53) (width 1) (layer F.Cu) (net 5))
 (segment (start 132.1 86.4) (end 131.05 86.4) (width 1) (layer F.Cu) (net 5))
 (segment (start 130.38 87.07) (end 130.38 87.53) (width 1) (layer F.Cu) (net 5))
 (segment (start 131.05 86.4) (end 130.38 87.07) (width 1) (layer F.Cu) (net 5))
 (segment (start 119.46 85.275) (end 119.47 85.285) (width 0.6) (layer F.Cu) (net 4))
 (segment (start 119.46 83.855) (end 119.46 85.275) (width 0.6) (layer F.Cu) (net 4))
 (segment (start 119.78501 85.60001) (end 121.95001 85.60001) (width 0.6) (layer F.Cu) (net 4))
 (segment (start 119.47 85.285) (end 119.78501 85.60001) (width 0.6) (layer F.Cu) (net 4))
 (segment (start 121.95001 85.60001) (end 124.385 88.035) (width 0.6) (layer F.Cu) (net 4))
 (segment (start 124.385 88.035) (end 125.3 88.95) (width 0.6) (layer F.Cu) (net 4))
 (segment (start 123.4 87.05) (end 124.385 88.035) (width 0.6) (layer F.Cu) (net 4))
 (segment (start 119.635 82.03) (end 119.46 82.205) (width 0.6) (layer F.Cu) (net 11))
 (segment (start 119.635 79.825) (end 119.635 82.03) (width 0.6) (layer F.Cu) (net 11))
 (segment (start 120.905 72.455) (end 119.95 71.5) (width 1) (layer F.Cu) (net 14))
 (segment (start 120.905 74.875) (end 120.905 72.455) (width 1) (layer F.Cu) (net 14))
 (segment (start 120.93 74.9) (end 120.45 74.9) (width 2.3) (layer F.Cu) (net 14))
 (segment (start 135 74.9) (end 120.93 74.9) (width 2.3) (layer F.Cu) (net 14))
 (segment (start 138.4575 83.08) (end 138.67 83.2925) (width 0.6) (layer F.Cu) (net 1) (status 1000000))
 (segment (start 136.9 83.08) (end 138.4575 83.08) (width 0.6) (layer F.Cu) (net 1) (status 1000000))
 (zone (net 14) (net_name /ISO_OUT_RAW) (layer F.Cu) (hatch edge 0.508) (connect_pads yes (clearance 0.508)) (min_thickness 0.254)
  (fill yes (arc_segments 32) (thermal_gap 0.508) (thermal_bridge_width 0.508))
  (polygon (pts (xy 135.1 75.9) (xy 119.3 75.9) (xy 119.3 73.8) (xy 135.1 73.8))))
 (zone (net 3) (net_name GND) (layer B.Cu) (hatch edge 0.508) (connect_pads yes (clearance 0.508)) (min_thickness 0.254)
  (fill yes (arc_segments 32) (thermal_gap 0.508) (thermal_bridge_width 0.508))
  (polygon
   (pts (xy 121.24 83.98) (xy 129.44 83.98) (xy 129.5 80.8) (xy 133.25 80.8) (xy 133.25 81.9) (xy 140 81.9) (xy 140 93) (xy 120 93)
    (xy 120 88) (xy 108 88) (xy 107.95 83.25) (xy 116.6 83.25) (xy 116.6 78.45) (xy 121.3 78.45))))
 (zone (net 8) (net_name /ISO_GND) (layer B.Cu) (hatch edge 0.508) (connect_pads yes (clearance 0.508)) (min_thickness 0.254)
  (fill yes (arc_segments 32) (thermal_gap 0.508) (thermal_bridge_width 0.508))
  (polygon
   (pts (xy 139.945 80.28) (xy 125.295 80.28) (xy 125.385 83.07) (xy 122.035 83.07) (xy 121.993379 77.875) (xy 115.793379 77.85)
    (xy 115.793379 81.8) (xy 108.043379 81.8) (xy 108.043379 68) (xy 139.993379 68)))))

